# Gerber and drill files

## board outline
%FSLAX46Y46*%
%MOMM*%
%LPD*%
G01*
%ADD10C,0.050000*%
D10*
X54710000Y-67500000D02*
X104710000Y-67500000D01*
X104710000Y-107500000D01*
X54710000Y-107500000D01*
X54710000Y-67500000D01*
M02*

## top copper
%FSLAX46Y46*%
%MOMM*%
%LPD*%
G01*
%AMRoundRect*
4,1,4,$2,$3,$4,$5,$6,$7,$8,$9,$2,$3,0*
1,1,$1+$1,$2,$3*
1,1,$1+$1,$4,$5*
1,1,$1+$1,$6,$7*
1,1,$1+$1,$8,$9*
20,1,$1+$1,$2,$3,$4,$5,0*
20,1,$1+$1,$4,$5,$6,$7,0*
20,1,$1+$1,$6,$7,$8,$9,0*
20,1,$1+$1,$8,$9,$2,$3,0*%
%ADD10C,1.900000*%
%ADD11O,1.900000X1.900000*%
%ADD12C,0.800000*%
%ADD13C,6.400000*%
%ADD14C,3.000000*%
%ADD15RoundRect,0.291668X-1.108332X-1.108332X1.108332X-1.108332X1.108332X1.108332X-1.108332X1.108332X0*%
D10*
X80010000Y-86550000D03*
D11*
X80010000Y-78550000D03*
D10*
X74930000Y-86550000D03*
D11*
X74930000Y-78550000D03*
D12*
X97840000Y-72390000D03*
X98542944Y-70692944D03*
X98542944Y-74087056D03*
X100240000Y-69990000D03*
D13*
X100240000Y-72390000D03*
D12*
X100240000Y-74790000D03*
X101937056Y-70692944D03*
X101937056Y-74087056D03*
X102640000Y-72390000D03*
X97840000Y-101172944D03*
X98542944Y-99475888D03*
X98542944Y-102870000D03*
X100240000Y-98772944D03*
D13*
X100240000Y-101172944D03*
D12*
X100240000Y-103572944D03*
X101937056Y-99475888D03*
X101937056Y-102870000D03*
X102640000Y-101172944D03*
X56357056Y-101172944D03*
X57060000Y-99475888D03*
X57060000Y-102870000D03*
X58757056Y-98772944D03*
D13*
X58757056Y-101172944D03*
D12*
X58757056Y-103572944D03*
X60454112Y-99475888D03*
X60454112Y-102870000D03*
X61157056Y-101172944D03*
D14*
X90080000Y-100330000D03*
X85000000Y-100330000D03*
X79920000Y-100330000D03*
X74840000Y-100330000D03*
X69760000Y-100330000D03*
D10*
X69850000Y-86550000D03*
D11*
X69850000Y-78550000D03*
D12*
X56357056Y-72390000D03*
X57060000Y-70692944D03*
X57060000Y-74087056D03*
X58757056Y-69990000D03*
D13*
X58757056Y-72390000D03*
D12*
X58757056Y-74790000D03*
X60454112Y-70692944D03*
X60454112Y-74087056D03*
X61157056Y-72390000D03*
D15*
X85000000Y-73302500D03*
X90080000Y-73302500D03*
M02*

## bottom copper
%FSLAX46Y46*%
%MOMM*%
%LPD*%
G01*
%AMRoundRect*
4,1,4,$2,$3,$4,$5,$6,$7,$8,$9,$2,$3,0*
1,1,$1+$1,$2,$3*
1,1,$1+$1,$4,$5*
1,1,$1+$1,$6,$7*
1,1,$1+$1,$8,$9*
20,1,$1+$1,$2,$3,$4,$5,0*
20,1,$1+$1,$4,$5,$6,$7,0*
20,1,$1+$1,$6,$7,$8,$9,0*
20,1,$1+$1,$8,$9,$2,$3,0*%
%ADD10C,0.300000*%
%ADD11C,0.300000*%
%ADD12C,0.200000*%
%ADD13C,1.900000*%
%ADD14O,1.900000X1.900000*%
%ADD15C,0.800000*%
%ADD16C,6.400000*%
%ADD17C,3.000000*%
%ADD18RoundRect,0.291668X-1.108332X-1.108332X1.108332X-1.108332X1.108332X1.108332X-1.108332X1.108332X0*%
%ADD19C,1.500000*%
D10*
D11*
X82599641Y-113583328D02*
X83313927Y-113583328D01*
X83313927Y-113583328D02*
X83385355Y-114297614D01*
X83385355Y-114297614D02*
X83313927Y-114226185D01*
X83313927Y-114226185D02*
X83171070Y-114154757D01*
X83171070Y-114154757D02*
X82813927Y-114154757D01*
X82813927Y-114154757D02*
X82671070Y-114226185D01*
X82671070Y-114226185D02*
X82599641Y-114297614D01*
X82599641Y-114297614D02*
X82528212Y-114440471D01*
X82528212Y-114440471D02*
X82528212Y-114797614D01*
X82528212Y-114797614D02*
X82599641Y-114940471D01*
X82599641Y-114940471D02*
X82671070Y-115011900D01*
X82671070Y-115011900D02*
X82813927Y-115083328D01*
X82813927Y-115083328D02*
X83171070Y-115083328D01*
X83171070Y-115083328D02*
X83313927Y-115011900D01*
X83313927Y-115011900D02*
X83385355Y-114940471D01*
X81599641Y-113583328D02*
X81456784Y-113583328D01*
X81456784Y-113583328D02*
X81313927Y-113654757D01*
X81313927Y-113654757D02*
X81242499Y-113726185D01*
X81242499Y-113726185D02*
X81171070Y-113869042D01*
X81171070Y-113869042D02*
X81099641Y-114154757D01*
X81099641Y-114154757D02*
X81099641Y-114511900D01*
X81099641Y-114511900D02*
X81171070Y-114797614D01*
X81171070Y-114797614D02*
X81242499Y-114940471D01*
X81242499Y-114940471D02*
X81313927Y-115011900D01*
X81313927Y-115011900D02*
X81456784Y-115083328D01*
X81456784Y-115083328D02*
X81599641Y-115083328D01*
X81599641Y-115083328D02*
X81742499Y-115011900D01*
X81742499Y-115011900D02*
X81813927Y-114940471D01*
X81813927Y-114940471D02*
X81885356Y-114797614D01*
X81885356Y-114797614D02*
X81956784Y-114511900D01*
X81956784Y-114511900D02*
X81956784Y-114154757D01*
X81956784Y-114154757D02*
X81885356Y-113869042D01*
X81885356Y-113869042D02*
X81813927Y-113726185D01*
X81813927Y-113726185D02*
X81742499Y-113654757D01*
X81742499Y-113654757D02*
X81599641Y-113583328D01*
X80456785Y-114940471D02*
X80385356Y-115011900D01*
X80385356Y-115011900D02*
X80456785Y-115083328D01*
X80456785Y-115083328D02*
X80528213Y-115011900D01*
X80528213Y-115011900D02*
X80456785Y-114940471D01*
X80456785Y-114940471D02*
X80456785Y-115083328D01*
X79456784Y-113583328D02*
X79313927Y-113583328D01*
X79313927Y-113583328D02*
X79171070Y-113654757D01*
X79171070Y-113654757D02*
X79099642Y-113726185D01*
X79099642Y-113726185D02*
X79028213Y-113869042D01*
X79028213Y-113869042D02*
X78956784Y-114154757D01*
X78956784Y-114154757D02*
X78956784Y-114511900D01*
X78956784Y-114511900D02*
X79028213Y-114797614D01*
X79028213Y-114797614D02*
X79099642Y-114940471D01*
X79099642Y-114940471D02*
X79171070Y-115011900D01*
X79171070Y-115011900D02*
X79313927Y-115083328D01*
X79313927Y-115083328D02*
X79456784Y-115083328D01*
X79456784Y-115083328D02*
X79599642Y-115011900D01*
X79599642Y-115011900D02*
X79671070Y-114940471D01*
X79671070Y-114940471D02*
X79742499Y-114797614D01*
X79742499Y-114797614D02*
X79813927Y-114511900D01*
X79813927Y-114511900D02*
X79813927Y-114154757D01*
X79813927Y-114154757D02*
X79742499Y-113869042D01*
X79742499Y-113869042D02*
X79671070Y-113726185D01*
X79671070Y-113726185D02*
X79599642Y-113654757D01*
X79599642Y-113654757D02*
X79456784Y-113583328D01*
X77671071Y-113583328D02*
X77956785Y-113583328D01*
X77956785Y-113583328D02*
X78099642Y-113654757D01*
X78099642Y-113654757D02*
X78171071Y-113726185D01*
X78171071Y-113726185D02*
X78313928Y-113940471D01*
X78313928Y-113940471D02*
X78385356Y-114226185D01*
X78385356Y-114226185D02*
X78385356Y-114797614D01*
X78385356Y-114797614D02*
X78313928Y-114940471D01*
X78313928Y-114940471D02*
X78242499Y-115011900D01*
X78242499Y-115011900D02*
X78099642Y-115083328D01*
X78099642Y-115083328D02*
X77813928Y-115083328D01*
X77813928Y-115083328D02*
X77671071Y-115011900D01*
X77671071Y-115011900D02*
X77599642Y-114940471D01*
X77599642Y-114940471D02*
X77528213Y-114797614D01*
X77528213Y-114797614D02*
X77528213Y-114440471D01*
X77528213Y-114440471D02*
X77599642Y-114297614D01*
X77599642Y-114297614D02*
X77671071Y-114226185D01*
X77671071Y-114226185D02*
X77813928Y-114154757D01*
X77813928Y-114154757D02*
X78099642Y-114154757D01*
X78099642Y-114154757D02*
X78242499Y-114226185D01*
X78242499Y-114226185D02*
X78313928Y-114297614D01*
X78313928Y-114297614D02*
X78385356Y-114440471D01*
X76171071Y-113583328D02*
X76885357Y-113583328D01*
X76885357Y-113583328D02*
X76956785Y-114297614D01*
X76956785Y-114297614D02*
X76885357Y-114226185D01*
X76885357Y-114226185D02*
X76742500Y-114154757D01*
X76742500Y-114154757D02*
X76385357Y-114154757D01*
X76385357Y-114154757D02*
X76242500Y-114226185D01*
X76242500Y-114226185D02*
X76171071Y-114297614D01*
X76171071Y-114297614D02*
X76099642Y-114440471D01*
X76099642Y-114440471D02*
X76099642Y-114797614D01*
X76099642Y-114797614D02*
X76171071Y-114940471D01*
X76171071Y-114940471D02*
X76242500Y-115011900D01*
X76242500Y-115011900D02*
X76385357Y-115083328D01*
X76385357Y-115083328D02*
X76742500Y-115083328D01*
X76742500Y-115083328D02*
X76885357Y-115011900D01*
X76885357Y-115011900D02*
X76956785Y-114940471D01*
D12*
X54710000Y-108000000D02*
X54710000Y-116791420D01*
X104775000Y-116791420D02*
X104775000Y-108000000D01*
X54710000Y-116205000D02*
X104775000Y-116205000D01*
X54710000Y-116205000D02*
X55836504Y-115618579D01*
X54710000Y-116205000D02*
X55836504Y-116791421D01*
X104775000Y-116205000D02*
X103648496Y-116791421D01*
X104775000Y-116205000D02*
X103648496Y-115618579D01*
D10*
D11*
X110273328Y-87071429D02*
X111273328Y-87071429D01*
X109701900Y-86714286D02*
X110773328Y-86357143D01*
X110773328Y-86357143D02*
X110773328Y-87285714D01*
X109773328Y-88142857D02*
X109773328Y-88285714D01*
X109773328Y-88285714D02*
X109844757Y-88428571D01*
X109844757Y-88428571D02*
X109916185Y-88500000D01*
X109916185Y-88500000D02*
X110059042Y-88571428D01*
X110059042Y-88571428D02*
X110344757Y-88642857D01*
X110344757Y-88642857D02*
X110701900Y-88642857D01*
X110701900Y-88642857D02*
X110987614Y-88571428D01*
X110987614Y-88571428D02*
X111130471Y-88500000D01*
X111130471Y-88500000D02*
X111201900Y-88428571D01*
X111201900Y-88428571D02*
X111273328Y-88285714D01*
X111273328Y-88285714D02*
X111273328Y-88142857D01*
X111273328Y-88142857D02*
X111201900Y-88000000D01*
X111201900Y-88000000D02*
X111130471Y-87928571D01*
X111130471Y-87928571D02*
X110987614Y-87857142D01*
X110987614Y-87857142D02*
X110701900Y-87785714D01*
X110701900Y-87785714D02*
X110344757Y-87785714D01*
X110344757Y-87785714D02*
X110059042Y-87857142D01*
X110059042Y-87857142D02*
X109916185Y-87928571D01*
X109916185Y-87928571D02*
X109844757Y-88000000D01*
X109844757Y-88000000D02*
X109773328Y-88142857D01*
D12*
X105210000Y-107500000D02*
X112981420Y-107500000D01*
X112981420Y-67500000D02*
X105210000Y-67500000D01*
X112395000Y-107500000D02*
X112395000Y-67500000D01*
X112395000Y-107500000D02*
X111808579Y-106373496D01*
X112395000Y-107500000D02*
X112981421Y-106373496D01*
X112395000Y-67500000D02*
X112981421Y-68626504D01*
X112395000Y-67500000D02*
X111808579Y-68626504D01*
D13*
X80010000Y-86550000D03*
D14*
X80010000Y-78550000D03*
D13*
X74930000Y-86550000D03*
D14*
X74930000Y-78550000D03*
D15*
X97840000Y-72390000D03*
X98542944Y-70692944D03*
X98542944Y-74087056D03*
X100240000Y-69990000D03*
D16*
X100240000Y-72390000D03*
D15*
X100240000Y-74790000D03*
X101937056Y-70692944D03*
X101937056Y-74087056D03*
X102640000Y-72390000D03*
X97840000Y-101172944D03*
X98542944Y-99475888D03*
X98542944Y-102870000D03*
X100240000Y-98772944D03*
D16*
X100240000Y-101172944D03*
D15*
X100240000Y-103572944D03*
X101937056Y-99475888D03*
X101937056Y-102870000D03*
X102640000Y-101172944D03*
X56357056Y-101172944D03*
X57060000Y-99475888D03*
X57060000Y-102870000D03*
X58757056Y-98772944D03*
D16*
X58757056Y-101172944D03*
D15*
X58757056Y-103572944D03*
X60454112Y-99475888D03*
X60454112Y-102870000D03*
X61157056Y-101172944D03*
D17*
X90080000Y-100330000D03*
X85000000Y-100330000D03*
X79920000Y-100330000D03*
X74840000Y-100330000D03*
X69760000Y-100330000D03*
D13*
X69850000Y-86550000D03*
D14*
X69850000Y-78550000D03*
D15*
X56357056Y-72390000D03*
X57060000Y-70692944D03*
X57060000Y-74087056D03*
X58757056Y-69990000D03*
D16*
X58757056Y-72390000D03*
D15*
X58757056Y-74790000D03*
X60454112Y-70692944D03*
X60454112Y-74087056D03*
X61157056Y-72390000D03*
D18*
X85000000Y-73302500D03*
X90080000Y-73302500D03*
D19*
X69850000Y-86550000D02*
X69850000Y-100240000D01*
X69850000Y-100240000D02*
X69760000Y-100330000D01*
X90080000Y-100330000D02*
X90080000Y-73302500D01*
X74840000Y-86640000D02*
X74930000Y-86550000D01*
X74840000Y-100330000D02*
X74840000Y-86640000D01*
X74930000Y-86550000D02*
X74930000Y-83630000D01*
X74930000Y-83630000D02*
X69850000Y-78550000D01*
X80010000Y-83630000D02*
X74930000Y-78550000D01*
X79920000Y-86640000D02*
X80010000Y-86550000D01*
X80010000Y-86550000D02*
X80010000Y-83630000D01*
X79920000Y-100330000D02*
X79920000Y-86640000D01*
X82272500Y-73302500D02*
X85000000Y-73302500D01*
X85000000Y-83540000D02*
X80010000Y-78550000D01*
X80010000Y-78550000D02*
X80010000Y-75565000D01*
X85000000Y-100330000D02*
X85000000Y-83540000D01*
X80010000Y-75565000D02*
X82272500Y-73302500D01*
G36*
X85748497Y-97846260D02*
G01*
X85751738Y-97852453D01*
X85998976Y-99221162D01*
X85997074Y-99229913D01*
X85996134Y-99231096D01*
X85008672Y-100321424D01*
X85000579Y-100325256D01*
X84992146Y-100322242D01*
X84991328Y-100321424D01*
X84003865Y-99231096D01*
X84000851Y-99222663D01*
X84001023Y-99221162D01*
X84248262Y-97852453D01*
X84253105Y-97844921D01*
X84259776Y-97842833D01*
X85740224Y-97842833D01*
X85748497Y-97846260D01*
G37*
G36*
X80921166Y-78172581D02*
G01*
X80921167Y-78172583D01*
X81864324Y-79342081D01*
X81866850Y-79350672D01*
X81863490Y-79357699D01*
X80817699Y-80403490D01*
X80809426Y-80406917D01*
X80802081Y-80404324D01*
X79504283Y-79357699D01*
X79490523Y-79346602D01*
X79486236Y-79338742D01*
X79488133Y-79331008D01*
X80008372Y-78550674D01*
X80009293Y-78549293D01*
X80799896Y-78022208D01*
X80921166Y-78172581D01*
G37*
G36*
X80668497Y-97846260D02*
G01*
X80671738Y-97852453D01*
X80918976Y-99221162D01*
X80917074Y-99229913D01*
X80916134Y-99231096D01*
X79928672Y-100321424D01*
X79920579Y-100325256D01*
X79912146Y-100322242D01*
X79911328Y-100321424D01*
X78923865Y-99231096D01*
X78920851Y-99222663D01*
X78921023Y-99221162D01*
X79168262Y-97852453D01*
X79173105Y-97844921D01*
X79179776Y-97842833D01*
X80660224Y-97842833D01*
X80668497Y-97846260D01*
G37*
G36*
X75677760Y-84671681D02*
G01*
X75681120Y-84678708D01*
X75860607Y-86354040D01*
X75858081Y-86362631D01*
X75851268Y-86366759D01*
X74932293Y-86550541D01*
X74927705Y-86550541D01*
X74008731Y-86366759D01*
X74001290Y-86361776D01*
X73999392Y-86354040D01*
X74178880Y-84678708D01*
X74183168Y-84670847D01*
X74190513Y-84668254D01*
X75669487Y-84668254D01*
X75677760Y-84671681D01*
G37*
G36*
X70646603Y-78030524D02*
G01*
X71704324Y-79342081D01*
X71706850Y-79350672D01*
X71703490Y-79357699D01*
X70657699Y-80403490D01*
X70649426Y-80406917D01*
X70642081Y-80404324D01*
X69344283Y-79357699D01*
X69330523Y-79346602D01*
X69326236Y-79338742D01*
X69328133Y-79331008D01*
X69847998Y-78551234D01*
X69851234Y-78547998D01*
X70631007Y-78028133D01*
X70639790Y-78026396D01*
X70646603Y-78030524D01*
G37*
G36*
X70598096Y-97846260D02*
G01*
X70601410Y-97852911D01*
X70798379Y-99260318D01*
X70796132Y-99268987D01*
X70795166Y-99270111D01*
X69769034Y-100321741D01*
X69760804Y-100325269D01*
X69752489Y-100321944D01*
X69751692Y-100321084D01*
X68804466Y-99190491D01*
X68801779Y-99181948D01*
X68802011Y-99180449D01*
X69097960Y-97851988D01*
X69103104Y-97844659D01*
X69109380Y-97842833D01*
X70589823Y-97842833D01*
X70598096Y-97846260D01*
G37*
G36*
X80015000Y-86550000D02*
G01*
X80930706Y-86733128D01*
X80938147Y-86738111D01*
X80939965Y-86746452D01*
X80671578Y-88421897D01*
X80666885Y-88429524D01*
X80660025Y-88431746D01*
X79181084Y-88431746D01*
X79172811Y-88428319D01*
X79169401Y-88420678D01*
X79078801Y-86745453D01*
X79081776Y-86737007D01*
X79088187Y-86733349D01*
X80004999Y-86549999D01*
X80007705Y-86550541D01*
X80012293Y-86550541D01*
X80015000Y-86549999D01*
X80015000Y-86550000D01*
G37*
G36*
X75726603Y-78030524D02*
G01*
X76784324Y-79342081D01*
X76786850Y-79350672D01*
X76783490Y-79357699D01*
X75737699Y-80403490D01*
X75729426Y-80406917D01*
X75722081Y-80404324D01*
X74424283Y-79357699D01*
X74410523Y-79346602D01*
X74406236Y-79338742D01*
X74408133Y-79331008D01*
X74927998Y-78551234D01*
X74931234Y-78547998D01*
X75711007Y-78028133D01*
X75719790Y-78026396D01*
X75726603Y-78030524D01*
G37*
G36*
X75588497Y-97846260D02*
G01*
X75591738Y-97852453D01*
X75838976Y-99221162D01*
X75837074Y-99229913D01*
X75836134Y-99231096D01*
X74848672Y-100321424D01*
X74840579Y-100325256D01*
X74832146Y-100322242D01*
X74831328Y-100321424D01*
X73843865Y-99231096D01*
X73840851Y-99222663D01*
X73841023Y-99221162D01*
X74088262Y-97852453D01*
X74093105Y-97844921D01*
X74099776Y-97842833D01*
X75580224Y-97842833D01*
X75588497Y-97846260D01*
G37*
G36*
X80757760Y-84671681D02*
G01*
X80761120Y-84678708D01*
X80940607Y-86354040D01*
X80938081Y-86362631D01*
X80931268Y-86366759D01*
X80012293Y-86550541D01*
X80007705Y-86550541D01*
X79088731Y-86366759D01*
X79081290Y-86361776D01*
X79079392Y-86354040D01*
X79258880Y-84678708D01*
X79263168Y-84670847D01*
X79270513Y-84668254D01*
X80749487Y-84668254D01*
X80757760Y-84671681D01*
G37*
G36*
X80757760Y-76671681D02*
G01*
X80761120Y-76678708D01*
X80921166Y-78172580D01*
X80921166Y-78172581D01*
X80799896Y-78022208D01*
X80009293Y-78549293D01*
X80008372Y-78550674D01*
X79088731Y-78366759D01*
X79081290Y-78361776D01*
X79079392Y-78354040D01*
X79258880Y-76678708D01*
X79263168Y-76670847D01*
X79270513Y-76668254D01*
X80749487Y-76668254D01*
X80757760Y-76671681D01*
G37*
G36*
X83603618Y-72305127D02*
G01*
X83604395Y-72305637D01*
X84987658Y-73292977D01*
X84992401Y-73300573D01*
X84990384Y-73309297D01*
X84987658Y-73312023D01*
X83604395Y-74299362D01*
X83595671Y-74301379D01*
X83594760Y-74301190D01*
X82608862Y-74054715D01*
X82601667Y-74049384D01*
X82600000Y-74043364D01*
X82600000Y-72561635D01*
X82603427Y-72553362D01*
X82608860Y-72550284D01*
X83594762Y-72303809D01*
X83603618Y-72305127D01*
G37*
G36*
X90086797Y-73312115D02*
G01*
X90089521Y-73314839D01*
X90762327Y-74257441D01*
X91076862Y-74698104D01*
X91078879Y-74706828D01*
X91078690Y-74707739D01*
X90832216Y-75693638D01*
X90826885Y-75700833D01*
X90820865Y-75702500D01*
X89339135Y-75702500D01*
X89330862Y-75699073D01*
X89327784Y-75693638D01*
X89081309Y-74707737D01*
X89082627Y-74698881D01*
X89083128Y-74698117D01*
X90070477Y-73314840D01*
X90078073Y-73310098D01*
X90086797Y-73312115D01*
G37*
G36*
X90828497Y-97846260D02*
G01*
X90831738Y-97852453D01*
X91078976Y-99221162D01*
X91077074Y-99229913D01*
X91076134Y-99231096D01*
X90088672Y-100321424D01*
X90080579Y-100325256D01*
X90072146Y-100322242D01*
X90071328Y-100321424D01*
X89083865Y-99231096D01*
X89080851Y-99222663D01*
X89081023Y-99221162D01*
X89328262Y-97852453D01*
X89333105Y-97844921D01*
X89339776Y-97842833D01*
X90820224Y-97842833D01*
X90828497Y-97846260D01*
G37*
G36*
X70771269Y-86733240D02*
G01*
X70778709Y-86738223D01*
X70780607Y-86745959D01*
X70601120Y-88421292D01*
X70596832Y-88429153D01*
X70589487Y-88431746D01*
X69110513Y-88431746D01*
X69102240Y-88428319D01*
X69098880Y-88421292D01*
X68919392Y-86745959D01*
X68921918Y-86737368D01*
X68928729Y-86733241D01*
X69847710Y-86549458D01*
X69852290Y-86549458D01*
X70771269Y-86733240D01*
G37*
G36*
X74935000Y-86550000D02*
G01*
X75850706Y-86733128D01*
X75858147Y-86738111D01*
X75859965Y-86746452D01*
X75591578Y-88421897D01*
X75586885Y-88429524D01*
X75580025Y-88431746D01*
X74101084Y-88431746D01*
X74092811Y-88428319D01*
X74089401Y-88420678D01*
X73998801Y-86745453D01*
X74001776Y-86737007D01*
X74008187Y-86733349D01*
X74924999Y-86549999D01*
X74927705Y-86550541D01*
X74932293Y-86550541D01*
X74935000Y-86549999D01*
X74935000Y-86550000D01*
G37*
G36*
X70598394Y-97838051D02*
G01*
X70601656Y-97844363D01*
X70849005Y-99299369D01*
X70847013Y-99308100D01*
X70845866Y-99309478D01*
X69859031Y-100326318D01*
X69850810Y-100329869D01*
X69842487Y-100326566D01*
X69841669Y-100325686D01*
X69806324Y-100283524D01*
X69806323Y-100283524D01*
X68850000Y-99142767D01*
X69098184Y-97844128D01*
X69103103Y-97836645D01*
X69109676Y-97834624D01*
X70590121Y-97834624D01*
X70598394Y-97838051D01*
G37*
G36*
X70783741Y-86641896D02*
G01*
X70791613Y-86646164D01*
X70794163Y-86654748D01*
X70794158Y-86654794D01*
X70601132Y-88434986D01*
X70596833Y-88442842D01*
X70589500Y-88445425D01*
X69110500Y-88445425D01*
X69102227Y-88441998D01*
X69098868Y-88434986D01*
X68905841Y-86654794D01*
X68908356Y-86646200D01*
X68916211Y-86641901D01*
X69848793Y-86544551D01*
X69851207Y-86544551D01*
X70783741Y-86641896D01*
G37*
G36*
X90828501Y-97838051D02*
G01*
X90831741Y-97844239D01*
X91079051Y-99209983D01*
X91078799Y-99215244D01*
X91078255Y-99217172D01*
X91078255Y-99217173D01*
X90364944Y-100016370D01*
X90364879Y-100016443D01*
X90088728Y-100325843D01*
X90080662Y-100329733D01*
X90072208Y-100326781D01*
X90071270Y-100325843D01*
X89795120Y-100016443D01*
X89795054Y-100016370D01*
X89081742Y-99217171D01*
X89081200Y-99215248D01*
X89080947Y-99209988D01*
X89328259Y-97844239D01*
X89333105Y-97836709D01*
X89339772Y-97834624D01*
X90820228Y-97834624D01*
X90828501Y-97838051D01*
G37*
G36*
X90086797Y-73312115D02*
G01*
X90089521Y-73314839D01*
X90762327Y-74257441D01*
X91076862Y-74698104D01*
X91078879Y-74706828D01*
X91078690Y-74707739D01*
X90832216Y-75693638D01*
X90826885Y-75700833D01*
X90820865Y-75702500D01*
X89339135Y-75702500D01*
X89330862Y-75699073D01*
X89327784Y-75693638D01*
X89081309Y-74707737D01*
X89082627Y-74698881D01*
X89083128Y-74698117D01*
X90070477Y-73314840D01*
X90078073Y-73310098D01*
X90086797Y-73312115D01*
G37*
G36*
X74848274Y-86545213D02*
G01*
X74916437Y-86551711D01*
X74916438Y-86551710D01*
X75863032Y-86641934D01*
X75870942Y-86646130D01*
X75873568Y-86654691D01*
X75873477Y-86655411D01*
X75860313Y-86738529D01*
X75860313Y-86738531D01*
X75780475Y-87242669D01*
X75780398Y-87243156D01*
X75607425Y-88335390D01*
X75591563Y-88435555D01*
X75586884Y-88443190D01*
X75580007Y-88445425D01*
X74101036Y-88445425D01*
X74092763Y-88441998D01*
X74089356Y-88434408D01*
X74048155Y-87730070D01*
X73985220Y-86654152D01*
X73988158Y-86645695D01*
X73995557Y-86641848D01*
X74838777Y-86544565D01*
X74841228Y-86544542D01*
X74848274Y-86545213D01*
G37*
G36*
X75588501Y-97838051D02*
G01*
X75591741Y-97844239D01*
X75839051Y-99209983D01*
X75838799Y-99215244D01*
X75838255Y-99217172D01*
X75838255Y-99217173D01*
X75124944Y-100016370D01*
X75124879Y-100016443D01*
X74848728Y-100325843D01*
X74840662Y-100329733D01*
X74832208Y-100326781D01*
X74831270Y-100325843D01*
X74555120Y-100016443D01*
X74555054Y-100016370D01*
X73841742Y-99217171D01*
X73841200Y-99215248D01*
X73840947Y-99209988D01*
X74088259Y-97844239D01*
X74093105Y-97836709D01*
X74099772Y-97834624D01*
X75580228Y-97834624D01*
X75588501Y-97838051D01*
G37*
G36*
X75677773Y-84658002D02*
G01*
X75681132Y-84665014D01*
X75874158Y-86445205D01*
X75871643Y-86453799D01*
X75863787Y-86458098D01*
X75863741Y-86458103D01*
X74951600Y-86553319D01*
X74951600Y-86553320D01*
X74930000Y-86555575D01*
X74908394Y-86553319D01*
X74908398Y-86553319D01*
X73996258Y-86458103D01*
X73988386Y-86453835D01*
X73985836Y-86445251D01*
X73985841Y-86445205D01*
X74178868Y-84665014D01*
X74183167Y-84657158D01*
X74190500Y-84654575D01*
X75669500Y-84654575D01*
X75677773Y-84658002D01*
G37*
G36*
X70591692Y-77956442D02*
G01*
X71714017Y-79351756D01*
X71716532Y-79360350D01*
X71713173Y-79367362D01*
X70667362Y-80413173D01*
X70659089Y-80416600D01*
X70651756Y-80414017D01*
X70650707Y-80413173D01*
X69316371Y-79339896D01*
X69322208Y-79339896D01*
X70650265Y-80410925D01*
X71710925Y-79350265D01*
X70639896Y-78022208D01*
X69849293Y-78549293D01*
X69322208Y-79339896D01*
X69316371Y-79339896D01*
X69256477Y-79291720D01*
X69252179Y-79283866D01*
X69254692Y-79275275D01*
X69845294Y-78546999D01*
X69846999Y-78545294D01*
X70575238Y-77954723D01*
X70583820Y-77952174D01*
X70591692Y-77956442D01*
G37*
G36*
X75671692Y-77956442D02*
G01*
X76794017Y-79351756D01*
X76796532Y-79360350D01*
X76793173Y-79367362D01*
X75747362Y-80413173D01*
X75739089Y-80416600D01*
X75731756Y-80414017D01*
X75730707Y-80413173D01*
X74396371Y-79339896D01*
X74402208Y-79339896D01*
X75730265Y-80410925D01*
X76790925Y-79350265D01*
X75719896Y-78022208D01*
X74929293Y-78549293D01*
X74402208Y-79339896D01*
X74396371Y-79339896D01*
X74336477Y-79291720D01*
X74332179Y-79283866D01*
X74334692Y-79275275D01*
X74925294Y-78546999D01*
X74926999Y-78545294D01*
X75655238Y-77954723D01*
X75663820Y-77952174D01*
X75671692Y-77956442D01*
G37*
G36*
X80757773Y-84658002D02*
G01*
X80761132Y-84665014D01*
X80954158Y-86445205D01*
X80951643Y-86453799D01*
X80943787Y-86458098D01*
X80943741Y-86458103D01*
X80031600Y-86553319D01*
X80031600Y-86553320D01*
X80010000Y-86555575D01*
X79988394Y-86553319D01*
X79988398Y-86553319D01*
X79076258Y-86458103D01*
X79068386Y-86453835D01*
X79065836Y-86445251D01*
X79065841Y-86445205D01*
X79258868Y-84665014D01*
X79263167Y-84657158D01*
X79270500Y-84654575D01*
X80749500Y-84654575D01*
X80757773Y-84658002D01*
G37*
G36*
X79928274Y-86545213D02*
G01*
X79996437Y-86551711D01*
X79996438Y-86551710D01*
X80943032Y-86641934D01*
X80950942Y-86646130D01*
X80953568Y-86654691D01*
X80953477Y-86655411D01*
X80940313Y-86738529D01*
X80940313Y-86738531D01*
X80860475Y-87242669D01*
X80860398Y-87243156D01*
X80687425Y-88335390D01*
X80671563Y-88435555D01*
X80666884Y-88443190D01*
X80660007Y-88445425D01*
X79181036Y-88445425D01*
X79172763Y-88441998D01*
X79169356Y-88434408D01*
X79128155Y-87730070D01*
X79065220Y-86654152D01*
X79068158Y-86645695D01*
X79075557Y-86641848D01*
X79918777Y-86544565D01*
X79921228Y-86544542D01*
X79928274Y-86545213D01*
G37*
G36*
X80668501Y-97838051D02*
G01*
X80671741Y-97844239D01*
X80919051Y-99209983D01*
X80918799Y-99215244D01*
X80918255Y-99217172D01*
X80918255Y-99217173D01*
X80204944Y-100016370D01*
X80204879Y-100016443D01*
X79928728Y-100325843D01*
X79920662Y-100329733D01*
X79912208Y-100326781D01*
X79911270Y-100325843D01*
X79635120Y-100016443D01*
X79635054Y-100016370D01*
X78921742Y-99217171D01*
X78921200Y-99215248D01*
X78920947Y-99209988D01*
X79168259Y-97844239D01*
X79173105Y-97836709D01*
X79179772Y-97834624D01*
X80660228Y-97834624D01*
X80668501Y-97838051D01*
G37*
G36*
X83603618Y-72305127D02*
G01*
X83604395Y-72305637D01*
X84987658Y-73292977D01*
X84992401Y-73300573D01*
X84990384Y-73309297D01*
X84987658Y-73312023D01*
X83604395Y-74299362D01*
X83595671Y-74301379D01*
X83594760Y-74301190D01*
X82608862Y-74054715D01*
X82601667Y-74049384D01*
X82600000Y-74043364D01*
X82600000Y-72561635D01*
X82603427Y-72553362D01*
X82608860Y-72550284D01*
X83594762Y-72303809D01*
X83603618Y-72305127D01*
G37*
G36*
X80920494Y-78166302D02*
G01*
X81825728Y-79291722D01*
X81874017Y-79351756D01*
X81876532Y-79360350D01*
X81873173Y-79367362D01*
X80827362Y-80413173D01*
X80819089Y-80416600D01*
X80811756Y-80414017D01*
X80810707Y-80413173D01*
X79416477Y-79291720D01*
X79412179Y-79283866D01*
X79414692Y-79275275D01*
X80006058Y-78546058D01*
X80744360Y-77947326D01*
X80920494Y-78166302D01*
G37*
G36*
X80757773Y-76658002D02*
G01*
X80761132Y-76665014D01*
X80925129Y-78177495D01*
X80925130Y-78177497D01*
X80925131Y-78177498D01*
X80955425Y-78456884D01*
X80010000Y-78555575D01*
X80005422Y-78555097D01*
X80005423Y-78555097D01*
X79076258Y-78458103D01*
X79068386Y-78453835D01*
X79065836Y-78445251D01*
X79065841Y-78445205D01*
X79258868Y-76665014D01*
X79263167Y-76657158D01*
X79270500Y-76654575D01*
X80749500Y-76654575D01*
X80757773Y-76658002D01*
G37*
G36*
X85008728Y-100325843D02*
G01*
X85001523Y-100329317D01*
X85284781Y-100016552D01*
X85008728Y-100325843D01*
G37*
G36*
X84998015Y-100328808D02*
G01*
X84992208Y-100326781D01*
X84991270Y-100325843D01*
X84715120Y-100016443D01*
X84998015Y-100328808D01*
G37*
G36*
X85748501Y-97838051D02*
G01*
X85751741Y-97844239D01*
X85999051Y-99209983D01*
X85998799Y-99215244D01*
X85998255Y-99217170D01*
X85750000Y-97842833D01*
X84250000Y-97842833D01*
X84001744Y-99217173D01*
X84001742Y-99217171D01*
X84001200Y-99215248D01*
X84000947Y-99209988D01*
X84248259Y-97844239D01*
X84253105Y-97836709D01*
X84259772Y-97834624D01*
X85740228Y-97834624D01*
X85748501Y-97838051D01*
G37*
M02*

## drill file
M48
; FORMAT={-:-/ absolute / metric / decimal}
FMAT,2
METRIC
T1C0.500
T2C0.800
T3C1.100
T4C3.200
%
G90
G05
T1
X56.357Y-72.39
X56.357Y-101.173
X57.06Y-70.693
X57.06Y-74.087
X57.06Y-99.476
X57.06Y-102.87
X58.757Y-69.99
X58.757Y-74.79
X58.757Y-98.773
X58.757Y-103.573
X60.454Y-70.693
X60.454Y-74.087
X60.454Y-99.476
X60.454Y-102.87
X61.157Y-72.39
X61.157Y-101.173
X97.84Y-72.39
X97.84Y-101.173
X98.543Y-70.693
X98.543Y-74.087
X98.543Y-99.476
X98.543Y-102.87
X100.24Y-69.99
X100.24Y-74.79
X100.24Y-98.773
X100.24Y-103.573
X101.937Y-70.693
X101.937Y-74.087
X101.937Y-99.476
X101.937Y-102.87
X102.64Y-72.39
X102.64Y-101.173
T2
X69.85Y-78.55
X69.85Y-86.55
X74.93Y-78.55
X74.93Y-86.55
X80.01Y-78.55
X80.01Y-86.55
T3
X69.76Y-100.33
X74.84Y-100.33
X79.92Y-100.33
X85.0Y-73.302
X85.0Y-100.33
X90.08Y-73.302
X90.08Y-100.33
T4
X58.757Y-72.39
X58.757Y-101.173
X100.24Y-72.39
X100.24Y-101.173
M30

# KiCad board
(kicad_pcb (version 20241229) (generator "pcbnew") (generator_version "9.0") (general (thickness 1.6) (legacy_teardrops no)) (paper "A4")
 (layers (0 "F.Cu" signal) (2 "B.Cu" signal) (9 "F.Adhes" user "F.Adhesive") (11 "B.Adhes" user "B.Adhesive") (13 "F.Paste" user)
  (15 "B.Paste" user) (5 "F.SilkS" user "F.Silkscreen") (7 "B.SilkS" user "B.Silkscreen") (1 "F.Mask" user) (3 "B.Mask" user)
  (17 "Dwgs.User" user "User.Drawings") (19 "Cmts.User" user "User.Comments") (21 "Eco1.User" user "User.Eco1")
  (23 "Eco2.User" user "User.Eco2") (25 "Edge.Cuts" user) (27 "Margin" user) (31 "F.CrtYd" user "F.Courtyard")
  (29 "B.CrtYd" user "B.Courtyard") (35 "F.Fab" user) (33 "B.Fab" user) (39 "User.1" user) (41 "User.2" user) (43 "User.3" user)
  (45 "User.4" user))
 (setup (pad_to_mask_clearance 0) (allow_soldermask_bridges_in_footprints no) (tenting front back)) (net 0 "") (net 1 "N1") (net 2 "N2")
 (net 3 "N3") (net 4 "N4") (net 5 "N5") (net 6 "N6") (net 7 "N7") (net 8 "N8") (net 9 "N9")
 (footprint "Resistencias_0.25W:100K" (layer "F.Cu") (at 80.01 86.55 90)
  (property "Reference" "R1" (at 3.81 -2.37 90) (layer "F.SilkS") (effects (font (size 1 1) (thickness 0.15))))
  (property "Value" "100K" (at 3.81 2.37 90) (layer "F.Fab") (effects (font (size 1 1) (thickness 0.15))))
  (pad "1" thru_hole circle (at 0 0 90) (size 1.9 1.9) (drill 0.8) (layers "*.Cu" "*.Mask") (remove_unused_layers no) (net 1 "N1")
   (teardrops (best_length_ratio 0.5) (max_length 1) (best_width_ratio 1) (max_width 2) (curved_edges no) (filter_ratio 0.9) (enabled yes)
    (allow_two_segments yes) (prefer_zone_connections yes)))
  (pad "2" thru_hole oval (at 8 0 90) (size 1.9 1.9) (drill 0.8) (layers "*.Cu" "*.Mask") (remove_unused_layers no) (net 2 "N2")
   (teardrops (best_length_ratio 0.5) (max_length 1) (best_width_ratio 1) (max_width 2) (curved_edges no) (filter_ratio 0.9) (enabled yes)
    (allow_two_segments yes) (prefer_zone_connections yes))))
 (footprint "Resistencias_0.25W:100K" (layer "F.Cu") (at 74.93 86.55 90)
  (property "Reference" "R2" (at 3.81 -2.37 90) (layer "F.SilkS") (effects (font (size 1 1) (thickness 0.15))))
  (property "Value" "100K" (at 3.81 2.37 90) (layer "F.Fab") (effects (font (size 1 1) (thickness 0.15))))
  (pad "1" thru_hole circle (at 0 0 90) (size 1.9 1.9) (drill 0.8) (layers "*.Cu" "*.Mask") (remove_unused_layers no) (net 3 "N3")
   (teardrops (best_length_ratio 0.5) (max_length 1) (best_width_ratio 1) (max_width 2) (curved_edges no) (filter_ratio 0.9) (enabled yes)
    (allow_two_segments yes) (prefer_zone_connections yes)))
  (pad "2" thru_hole oval (at 8 0 90) (size 1.9 1.9) (drill 0.8) (layers "*.Cu" "*.Mask") (remove_unused_layers no) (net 1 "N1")
   (teardrops (best_length_ratio 0.5) (max_length 1) (best_width_ratio 1) (max_width 2) (curved_edges no) (filter_ratio 0.9) (enabled yes)
    (allow_two_segments yes) (prefer_zone_connections yes))))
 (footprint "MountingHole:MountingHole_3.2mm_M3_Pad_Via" (layer "F.Cu") (at 100.24 72.39)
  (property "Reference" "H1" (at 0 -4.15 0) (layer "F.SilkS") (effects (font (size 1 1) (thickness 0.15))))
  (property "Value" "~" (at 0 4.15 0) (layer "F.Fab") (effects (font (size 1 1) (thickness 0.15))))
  (pad "1" thru_hole circle (at -2.4 0) (size 0.8 0.8) (drill 0.5) (layers "*.Cu" "*.Mask") (remove_unused_layers no) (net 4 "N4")
   (zone_connect 2)
   (teardrops (best_length_ratio 0.5) (max_length 1) (best_width_ratio 1) (max_width 2) (curved_edges no) (filter_ratio 0.9) (enabled yes)
    (allow_two_segments yes) (prefer_zone_connections yes)))
  (pad "1" thru_hole circle (at -1.697056 -1.697056) (size 0.8 0.8) (drill 0.5) (layers "*.Cu" "*.Mask") (remove_unused_layers no)
   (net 4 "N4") (zone_connect 2)
   (teardrops (best_length_ratio 0.5) (max_length 1) (best_width_ratio 1) (max_width 2) (curved_edges no) (filter_ratio 0.9) (enabled yes)
    (allow_two_segments yes) (prefer_zone_connections yes)))
  (pad "1" thru_hole circle (at -1.697056 1.697056) (size 0.8 0.8) (drill 0.5) (layers "*.Cu" "*.Mask") (remove_unused_layers no)
   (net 4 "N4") (zone_connect 2)
   (teardrops (best_length_ratio 0.5) (max_length 1) (best_width_ratio 1) (max_width 2) (curved_edges no) (filter_ratio 0.9) (enabled yes)
    (allow_two_segments yes) (prefer_zone_connections yes)))
  (pad "1" thru_hole circle (at 0 -2.4) (size 0.8 0.8) (drill 0.5) (layers "*.Cu" "*.Mask") (remove_unused_layers no) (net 4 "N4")
   (zone_connect 2)
   (teardrops (best_length_ratio 0.5) (max_length 1) (best_width_ratio 1) (max_width 2) (curved_edges no) (filter_ratio 0.9) (enabled yes)
    (allow_two_segments yes) (prefer_zone_connections yes)))
  (pad "1" thru_hole circle (at 0 0) (size 6.4 6.4) (drill 3.2) (layers "*.Cu" "*.Mask") (remove_unused_layers no) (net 4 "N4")
   (zone_connect 2)
   (teardrops (best_length_ratio 0.5) (max_length 1) (best_width_ratio 1) (max_width 2) (curved_edges no) (filter_ratio 0.9) (enabled yes)
    (allow_two_segments yes) (prefer_zone_connections yes)))
  (pad "1" thru_hole circle (at 0 2.4) (size 0.8 0.8) (drill 0.5) (layers "*.Cu" "*.Mask") (remove_unused_layers no) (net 4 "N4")
   (zone_connect 2)
   (teardrops (best_length_ratio 0.5) (max_length 1) (best_width_ratio 1) (max_width 2) (curved_edges no) (filter_ratio 0.9) (enabled yes)
    (allow_two_segments yes) (prefer_zone_connections yes)))
  (pad "1" thru_hole circle (at 1.697056 -1.697056) (size 0.8 0.8) (drill 0.5) (layers "*.Cu" "*.Mask") (remove_unused_layers no)
   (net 4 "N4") (zone_connect 2)
   (teardrops (best_length_ratio 0.5) (max_length 1) (best_width_ratio 1) (max_width 2) (curved_edges no) (filter_ratio 0.9) (enabled yes)
    (allow_two_segments yes) (prefer_zone_connections yes)))
  (pad "1" thru_hole circle (at 1.697056 1.697056) (size 0.8 0.8) (drill 0.5) (layers "*.Cu" "*.Mask") (remove_unused_layers no)
   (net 4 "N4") (zone_connect 2)
   (teardrops (best_length_ratio 0.5) (max_length 1) (best_width_ratio 1) (max_width 2) (curved_edges no) (filter_ratio 0.9) (enabled yes)
    (allow_two_segments yes) (prefer_zone_connections yes)))
  (pad "1" thru_hole circle (at 2.4 0) (size 0.8 0.8) (drill 0.5) (layers "*.Cu" "*.Mask") (remove_unused_layers no) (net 4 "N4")
   (zone_connect 2)
   (teardrops (best_length_ratio 0.5) (max_length 1) (best_width_ratio 1) (max_width 2) (curved_edges no) (filter_ratio 0.9) (enabled yes)
    (allow_two_segments yes) (prefer_zone_connections yes))))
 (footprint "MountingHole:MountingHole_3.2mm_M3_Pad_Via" (layer "F.Cu") (at 100.24 101.172944)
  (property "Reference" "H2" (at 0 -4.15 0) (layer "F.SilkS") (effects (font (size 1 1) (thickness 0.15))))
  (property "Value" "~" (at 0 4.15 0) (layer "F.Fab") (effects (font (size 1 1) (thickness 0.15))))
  (pad "1" thru_hole circle (at -2.4 0) (size 0.8 0.8) (drill 0.5) (layers "*.Cu" "*.Mask") (remove_unused_layers no) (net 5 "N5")
   (zone_connect 2)
   (teardrops (best_length_ratio 0.5) (max_length 1) (best_width_ratio 1) (max_width 2) (curved_edges no) (filter_ratio 0.9) (enabled yes)
    (allow_two_segments yes) (prefer_zone_connections yes)))
  (pad "1" thru_hole circle (at -1.697056 -1.697056) (size 0.8 0.8) (drill 0.5) (layers "*.Cu" "*.Mask") (remove_unused_layers no)
   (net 5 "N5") (zone_connect 2)
   (teardrops (best_length_ratio 0.5) (max_length 1) (best_width_ratio 1) (max_width 2) (curved_edges no) (filter_ratio 0.9) (enabled yes)
    (allow_two_segments yes) (prefer_zone_connections yes)))
  (pad "1" thru_hole circle (at -1.697056 1.697056) (size 0.8 0.8) (drill 0.5) (layers "*.Cu" "*.Mask") (remove_unused_layers no)
   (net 5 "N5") (zone_connect 2)
   (teardrops (best_length_ratio 0.5) (max_length 1) (best_width_ratio 1) (max_width 2) (curved_edges no) (filter_ratio 0.9) (enabled yes)
    (allow_two_segments yes) (prefer_zone_connections yes)))
  (pad "1" thru_hole circle (at 0 -2.4) (size 0.8 0.8) (drill 0.5) (layers "*.Cu" "*.Mask") (remove_unused_layers no) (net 5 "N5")
   (zone_connect 2)
   (teardrops (best_length_ratio 0.5) (max_length 1) (best_width_ratio 1) (max_width 2) (curved_edges no) (filter_ratio 0.9) (enabled yes)
    (allow_two_segments yes) (prefer_zone_connections yes)))
  (pad "1" thru_hole circle (at 0 0) (size 6.4 6.4) (drill 3.2) (layers "*.Cu" "*.Mask") (remove_unused_layers no) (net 5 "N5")
   (zone_connect 2)
   (teardrops (best_length_ratio 0.5) (max_length 1) (best_width_ratio 1) (max_width 2) (curved_edges no) (filter_ratio 0.9) (enabled yes)
    (allow_two_segments yes) (prefer_zone_connections yes)))
  (pad "1" thru_hole circle (at 0 2.4) (size 0.8 0.8) (drill 0.5) (layers "*.Cu" "*.Mask") (remove_unused_layers no) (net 5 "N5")
   (zone_connect 2)
   (teardrops (best_length_ratio 0.5) (max_length 1) (best_width_ratio 1) (max_width 2) (curved_edges no) (filter_ratio 0.9) (enabled yes)
    (allow_two_segments yes) (prefer_zone_connections yes)))
  (pad "1" thru_hole circle (at 1.697056 -1.697056) (size 0.8 0.8) (drill 0.5) (layers "*.Cu" "*.Mask") (remove_unused_layers no)
   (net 5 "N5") (zone_connect 2)
   (teardrops (best_length_ratio 0.5) (max_length 1) (best_width_ratio 1) (max_width 2) (curved_edges no) (filter_ratio 0.9) (enabled yes)
    (allow_two_segments yes) (prefer_zone_connections yes)))
  (pad "1" thru_hole circle (at 1.697056 1.697056) (size 0.8 0.8) (drill 0.5) (layers "*.Cu" "*.Mask") (remove_unused_layers no)
   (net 5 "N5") (zone_connect 2)
   (teardrops (best_length_ratio 0.5) (max_length 1) (best_width_ratio 1) (max_width 2) (curved_edges no) (filter_ratio 0.9) (enabled yes)
    (allow_two_segments yes) (prefer_zone_connections yes)))
  (pad "1" thru_hole circle (at 2.4 0) (size 0.8 0.8) (drill 0.5) (layers "*.Cu" "*.Mask") (remove_unused_layers no) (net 5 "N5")
   (zone_connect 2)
   (teardrops (best_length_ratio 0.5) (max_length 1) (best_width_ratio 1) (max_width 2) (curved_edges no) (filter_ratio 0.9) (enabled yes)
    (allow_two_segments yes) (prefer_zone_connections yes))))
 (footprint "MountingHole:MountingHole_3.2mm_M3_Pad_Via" (layer "F.Cu") (at 58.757056 101.172944)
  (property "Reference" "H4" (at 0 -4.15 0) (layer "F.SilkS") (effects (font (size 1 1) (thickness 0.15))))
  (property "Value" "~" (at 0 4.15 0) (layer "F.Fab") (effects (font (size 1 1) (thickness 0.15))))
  (pad "1" thru_hole circle (at -2.4 0) (size 0.8 0.8) (drill 0.5) (layers "*.Cu" "*.Mask") (remove_unused_layers no) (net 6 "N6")
   (zone_connect 2)
   (teardrops (best_length_ratio 0.5) (max_length 1) (best_width_ratio 1) (max_width 2) (curved_edges no) (filter_ratio 0.9) (enabled yes)
    (allow_two_segments yes) (prefer_zone_connections yes)))
  (pad "1" thru_hole circle (at -1.697056 -1.697056) (size 0.8 0.8) (drill 0.5) (layers "*.Cu" "*.Mask") (remove_unused_layers no)
   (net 6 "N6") (zone_connect 2)
   (teardrops (best_length_ratio 0.5) (max_length 1) (best_width_ratio 1) (max_width 2) (curved_edges no) (filter_ratio 0.9) (enabled yes)
    (allow_two_segments yes) (prefer_zone_connections yes)))
  (pad "1" thru_hole circle (at -1.697056 1.697056) (size 0.8 0.8) (drill 0.5) (layers "*.Cu" "*.Mask") (remove_unused_layers no)
   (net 6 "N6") (zone_connect 2)
   (teardrops (best_length_ratio 0.5) (max_length 1) (best_width_ratio 1) (max_width 2) (curved_edges no) (filter_ratio 0.9) (enabled yes)
    (allow_two_segments yes) (prefer_zone_connections yes)))
  (pad "1" thru_hole circle (at 0 -2.4) (size 0.8 0.8) (drill 0.5) (layers "*.Cu" "*.Mask") (remove_unused_layers no) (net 6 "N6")
   (zone_connect 2)
   (teardrops (best_length_ratio 0.5) (max_length 1) (best_width_ratio 1) (max_width 2) (curved_edges no) (filter_ratio 0.9) (enabled yes)
    (allow_two_segments yes) (prefer_zone_connections yes)))
  (pad "1" thru_hole circle (at 0 0) (size 6.4 6.4) (drill 3.2) (layers "*.Cu" "*.Mask") (remove_unused_layers no) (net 6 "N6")
   (zone_connect 2)
   (teardrops (best_length_ratio 0.5) (max_length 1) (best_width_ratio 1) (max_width 2) (curved_edges no) (filter_ratio 0.9) (enabled yes)
    (allow_two_segments yes) (prefer_zone_connections yes)))
  (pad "1" thru_hole circle (at 0 2.4) (size 0.8 0.8) (drill 0.5) (layers "*.Cu" "*.Mask") (remove_unused_layers no) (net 6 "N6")
   (zone_connect 2)
   (teardrops (best_length_ratio 0.5) (max_length 1) (best_width_ratio 1) (max_width 2) (curved_edges no) (filter_ratio 0.9) (enabled yes)
    (allow_two_segments yes) (prefer_zone_connections yes)))
  (pad "1" thru_hole circle (at 1.697056 -1.697056) (size 0.8 0.8) (drill 0.5) (layers "*.Cu" "*.Mask") (remove_unused_layers no)
   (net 6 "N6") (zone_connect 2)
   (teardrops (best_length_ratio 0.5) (max_length 1) (best_width_ratio 1) (max_width 2) (curved_edges no) (filter_ratio 0.9) (enabled yes)
    (allow_two_segments yes) (prefer_zone_connections yes)))
  (pad "1" thru_hole circle (at 1.697056 1.697056) (size 0.8 0.8) (drill 0.5) (layers "*.Cu" "*.Mask") (remove_unused_layers no)
   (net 6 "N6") (zone_connect 2)
   (teardrops (best_length_ratio 0.5) (max_length 1) (best_width_ratio 1) (max_width 2) (curved_edges no) (filter_ratio 0.9) (enabled yes)
    (allow_two_segments yes) (prefer_zone_connections yes)))
  (pad "1" thru_hole circle (at 2.4 0) (size 0.8 0.8) (drill 0.5) (layers "*.Cu" "*.Mask") (remove_unused_layers no) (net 6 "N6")
   (zone_connect 2)
   (teardrops (best_length_ratio 0.5) (max_length 1) (best_width_ratio 1) (max_width 2) (curved_edges no) (filter_ratio 0.9) (enabled yes)
    (allow_two_segments yes) (prefer_zone_connections yes))))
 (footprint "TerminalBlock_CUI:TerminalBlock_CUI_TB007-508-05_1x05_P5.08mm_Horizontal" (layer "F.Cu") (at 90.08 100.33 180)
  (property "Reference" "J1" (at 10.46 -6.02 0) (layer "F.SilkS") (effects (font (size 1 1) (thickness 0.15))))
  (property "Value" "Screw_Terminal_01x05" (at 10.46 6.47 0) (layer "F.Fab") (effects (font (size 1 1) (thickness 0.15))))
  (pad "1" thru_hole circle (at 0 0 180) (size 3 3) (drill 1.1) (layers "*.Cu" "*.Mask") (remove_unused_layers no) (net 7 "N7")
   (teardrops (best_length_ratio 0.5) (max_length 1) (best_width_ratio 1) (max_width 2) (curved_edges no) (filter_ratio 0.9) (enabled yes)
    (allow_two_segments yes) (prefer_zone_connections yes)))
  (pad "2" thru_hole circle (at 5.08 0 180) (size 3 3) (drill 1.1) (layers "*.Cu" "*.Mask") (remove_unused_layers no) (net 2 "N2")
   (teardrops (best_length_ratio 0.5) (max_length 1) (best_width_ratio 1) (max_width 2) (curved_edges no) (filter_ratio 0.9) (enabled yes)
    (allow_two_segments yes) (prefer_zone_connections yes)))
  (pad "3" thru_hole circle (at 10.16 0 180) (size 3 3) (drill 1.1) (layers "*.Cu" "*.Mask") (remove_unused_layers no) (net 1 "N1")
   (teardrops (best_length_ratio 0.5) (max_length 1) (best_width_ratio 1) (max_width 2) (curved_edges no) (filter_ratio 0.9) (enabled yes)
    (allow_two_segments yes) (prefer_zone_connections yes)))
  (pad "4" thru_hole circle (at 15.24 0 180) (size 3 3) (drill 1.1) (layers "*.Cu" "*.Mask") (remove_unused_layers no) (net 3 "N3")
   (teardrops (best_length_ratio 0.5) (max_length 1) (best_width_ratio 1) (max_width 2) (curved_edges no) (filter_ratio 0.9) (enabled yes)
    (allow_two_segments yes) (prefer_zone_connections yes)))
  (pad "5" thru_hole circle (at 20.32 0 180) (size 3 3) (drill 1.1) (layers "*.Cu" "*.Mask") (remove_unused_layers no) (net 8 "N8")
   (teardrops (best_length_ratio 0.5) (max_length 1) (best_width_ratio 1) (max_width 2) (curved_edges no) (filter_ratio 0.9) (enabled yes)
    (allow_two_segments yes) (prefer_zone_connections yes))))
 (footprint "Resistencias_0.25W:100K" (layer "F.Cu") (at 69.85 86.55 90)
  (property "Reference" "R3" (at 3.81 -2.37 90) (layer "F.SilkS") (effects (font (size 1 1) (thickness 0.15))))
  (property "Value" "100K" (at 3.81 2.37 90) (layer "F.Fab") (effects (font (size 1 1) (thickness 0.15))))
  (pad "1" thru_hole circle (at 0 0 90) (size 1.9 1.9) (drill 0.8) (layers "*.Cu" "*.Mask") (remove_unused_layers no) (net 8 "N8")
   (teardrops (best_length_ratio 0.5) (max_length 1) (best_width_ratio 1) (max_width 2) (curved_edges no) (filter_ratio 0.9) (enabled yes)
    (allow_two_segments yes) (prefer_zone_connections yes)))
  (pad "2" thru_hole oval (at 8 0 90) (size 1.9 1.9) (drill 0.8) (layers "*.Cu" "*.Mask") (remove_unused_layers no) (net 3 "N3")
   (teardrops (best_length_ratio 0.5) (max_length 1) (best_width_ratio 1) (max_width 2) (curved_edges no) (filter_ratio 0.9) (enabled yes)
    (allow_two_segments yes) (prefer_zone_connections yes))))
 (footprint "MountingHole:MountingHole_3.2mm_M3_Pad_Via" (layer "F.Cu") (at 58.757056 72.39)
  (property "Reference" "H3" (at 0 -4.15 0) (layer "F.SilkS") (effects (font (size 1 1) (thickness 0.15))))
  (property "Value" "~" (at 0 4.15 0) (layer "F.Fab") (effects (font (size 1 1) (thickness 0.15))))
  (pad "1" thru_hole circle (at -2.4 0) (size 0.8 0.8) (drill 0.5) (layers "*.Cu" "*.Mask") (remove_unused_layers no) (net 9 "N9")
   (zone_connect 2)
   (teardrops (best_length_ratio 0.5) (max_length 1) (best_width_ratio 1) (max_width 2) (curved_edges no) (filter_ratio 0.9) (enabled yes)
    (allow_two_segments yes) (prefer_zone_connections yes)))
  (pad "1" thru_hole circle (at -1.697056 -1.697056) (size 0.8 0.8) (drill 0.5) (layers "*.Cu" "*.Mask") (remove_unused_layers no)
   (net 9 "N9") (zone_connect 2)
   (teardrops (best_length_ratio 0.5) (max_length 1) (best_width_ratio 1) (max_width 2) (curved_edges no) (filter_ratio 0.9) (enabled yes)
    (allow_two_segments yes) (prefer_zone_connections yes)))
  (pad "1" thru_hole circle (at -1.697056 1.697056) (size 0.8 0.8) (drill 0.5) (layers "*.Cu" "*.Mask") (remove_unused_layers no)
   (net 9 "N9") (zone_connect 2)
   (teardrops (best_length_ratio 0.5) (max_length 1) (best_width_ratio 1) (max_width 2) (curved_edges no) (filter_ratio 0.9) (enabled yes)
    (allow_two_segments yes) (prefer_zone_connections yes)))
  (pad "1" thru_hole circle (at 0 -2.4) (size 0.8 0.8) (drill 0.5) (layers "*.Cu" "*.Mask") (remove_unused_layers no) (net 9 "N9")
   (zone_connect 2)
   (teardrops (best_length_ratio 0.5) (max_length 1) (best_width_ratio 1) (max_width 2) (curved_edges no) (filter_ratio 0.9) (enabled yes)
    (allow_two_segments yes) (prefer_zone_connections yes)))
  (pad "1" thru_hole circle (at 0 0) (size 6.4 6.4) (drill 3.2) (layers "*.Cu" "*.Mask") (remove_unused_layers no) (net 9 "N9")
   (zone_connect 2)
   (teardrops (best_length_ratio 0.5) (max_length 1) (best_width_ratio 1) (max_width 2) (curved_edges no) (filter_ratio 0.9) (enabled yes)
    (allow_two_segments yes) (prefer_zone_connections yes)))
  (pad "1" thru_hole circle (at 0 2.4) (size 0.8 0.8) (drill 0.5) (layers "*.Cu" "*.Mask") (remove_unused_layers no) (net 9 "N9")
   (zone_connect 2)
   (teardrops (best_length_ratio 0.5) (max_length 1) (best_width_ratio 1) (max_width 2) (curved_edges no) (filter_ratio 0.9) (enabled yes)
    (allow_two_segments yes) (prefer_zone_connections yes)))
  (pad "1" thru_hole circle (at 1.697056 -1.697056) (size 0.8 0.8) (drill 0.5) (layers "*.Cu" "*.Mask") (remove_unused_layers no)
   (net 9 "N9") (zone_connect 2)
   (teardrops (best_length_ratio 0.5) (max_length 1) (best_width_ratio 1) (max_width 2) (curved_edges no) (filter_ratio 0.9) (enabled yes)
    (allow_two_segments yes) (prefer_zone_connections yes)))
  (pad "1" thru_hole circle (at 1.697056 1.697056) (size 0.8 0.8) (drill 0.5) (layers "*.Cu" "*.Mask") (remove_unused_layers no)
   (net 9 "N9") (zone_connect 2)
   (teardrops (best_length_ratio 0.5) (max_length 1) (best_width_ratio 1) (max_width 2) (curved_edges no) (filter_ratio 0.9) (enabled yes)
    (allow_two_segments yes) (prefer_zone_connections yes)))
  (pad "1" thru_hole circle (at 2.4 0) (size 0.8 0.8) (drill 0.5) (layers "*.Cu" "*.Mask") (remove_unused_layers no) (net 9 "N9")
   (zone_connect 2)
   (teardrops (best_length_ratio 0.5) (max_length 1) (best_width_ratio 1) (max_width 2) (curved_edges no) (filter_ratio 0.9) (enabled yes)
    (allow_two_segments yes) (prefer_zone_connections yes))))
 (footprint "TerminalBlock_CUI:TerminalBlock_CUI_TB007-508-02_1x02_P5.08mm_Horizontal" (layer "F.Cu") (at 85 73.3025)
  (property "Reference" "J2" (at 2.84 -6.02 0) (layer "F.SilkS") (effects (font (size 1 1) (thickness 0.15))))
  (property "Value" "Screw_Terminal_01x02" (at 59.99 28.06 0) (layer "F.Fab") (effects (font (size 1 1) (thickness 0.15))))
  (pad "1" thru_hole roundrect (at 0 0) (size 2.8 2.8) (drill 1.1) (layers "*.Cu" "*.Mask") (remove_unused_layers no)
   (roundrect_rratio 0.104167) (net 2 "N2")
   (teardrops (best_length_ratio 0.5) (max_length 1) (best_width_ratio 1) (max_width 2) (curved_edges no) (filter_ratio 0.9) (enabled yes)
    (allow_two_segments yes) (prefer_zone_connections yes)))
  (pad "2" thru_hole roundrect (at 5.08 0) (size 2.8 2.8) (drill 1.1) (layers "*.Cu" "*.Mask") (remove_unused_layers no)
   (roundrect_rratio 0.104167) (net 7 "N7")
   (teardrops (best_length_ratio 0.5) (max_length 1) (best_width_ratio 1) (max_width 2) (curved_edges no) (filter_ratio 0.9) (enabled yes)
    (allow_two_segments yes) (prefer_zone_connections yes))))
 (gr_rect (start 54.71 67.5) (end 104.71 107.5) (stroke (width 0.05) (type default)) (fill no) (layer "Edge.Cuts"))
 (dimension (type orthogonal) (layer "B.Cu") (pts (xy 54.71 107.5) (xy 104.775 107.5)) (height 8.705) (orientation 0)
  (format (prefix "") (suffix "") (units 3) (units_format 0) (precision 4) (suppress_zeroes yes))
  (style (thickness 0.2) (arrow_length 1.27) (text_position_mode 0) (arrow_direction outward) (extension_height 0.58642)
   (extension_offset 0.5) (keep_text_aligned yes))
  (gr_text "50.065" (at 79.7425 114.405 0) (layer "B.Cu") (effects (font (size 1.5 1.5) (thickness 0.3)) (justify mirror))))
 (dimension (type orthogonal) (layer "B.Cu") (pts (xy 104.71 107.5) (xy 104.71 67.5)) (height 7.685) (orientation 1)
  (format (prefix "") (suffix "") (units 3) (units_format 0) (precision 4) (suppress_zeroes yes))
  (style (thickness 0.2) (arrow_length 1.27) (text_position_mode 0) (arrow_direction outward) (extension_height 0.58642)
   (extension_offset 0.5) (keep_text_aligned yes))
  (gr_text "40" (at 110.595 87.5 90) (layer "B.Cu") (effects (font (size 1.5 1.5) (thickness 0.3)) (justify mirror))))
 (segment (start 69.85 86.55) (end 69.85 100.24) (width 1.5) (layer "B.Cu") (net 8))
 (segment (start 69.85 100.24) (end 69.76 100.33) (width 1.5) (layer "B.Cu") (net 8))
 (segment (start 90.08 100.33) (end 90.08 73.3025) (width 1.5) (layer "B.Cu") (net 7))
 (segment (start 74.84 86.64) (end 74.93 86.55) (width 1.5) (layer "B.Cu") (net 3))
 (segment (start 74.84 100.33) (end 74.84 86.64) (width 1.5) (layer "B.Cu") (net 3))
 (segment (start 74.93 86.55) (end 74.93 83.63) (width 1.5) (layer "B.Cu") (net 3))
 (segment (start 74.93 83.63) (end 69.85 78.55) (width 1.5) (layer "B.Cu") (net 3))
 (segment (start 80.01 83.63) (end 74.93 78.55) (width 1.5) (layer "B.Cu") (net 1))
 (segment (start 79.92 86.64) (end 80.01 86.55) (width 1.5) (layer "B.Cu") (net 1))
 (segment (start 80.01 86.55) (end 80.01 83.63) (width 1.5) (layer "B.Cu") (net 1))
 (segment (start 79.92 100.33) (end 79.92 86.64) (width 1.5) (layer "B.Cu") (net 1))
 (segment (start 82.2725 73.3025) (end 85 73.3025) (width 1.5) (layer "B.Cu") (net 2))
 (segment (start 85 83.54) (end 80.01 78.55) (width 1.5) (layer "B.Cu") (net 2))
 (segment (start 80.01 78.55) (end 80.01 75.565) (width 1.5) (layer "B.Cu") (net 2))
 (segment (start 85 100.33) (end 85 83.54) (width 1.5) (layer "B.Cu") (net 2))
 (segment (start 80.01 75.565) (end 82.2725 73.3025) (width 1.5) (layer "B.Cu") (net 2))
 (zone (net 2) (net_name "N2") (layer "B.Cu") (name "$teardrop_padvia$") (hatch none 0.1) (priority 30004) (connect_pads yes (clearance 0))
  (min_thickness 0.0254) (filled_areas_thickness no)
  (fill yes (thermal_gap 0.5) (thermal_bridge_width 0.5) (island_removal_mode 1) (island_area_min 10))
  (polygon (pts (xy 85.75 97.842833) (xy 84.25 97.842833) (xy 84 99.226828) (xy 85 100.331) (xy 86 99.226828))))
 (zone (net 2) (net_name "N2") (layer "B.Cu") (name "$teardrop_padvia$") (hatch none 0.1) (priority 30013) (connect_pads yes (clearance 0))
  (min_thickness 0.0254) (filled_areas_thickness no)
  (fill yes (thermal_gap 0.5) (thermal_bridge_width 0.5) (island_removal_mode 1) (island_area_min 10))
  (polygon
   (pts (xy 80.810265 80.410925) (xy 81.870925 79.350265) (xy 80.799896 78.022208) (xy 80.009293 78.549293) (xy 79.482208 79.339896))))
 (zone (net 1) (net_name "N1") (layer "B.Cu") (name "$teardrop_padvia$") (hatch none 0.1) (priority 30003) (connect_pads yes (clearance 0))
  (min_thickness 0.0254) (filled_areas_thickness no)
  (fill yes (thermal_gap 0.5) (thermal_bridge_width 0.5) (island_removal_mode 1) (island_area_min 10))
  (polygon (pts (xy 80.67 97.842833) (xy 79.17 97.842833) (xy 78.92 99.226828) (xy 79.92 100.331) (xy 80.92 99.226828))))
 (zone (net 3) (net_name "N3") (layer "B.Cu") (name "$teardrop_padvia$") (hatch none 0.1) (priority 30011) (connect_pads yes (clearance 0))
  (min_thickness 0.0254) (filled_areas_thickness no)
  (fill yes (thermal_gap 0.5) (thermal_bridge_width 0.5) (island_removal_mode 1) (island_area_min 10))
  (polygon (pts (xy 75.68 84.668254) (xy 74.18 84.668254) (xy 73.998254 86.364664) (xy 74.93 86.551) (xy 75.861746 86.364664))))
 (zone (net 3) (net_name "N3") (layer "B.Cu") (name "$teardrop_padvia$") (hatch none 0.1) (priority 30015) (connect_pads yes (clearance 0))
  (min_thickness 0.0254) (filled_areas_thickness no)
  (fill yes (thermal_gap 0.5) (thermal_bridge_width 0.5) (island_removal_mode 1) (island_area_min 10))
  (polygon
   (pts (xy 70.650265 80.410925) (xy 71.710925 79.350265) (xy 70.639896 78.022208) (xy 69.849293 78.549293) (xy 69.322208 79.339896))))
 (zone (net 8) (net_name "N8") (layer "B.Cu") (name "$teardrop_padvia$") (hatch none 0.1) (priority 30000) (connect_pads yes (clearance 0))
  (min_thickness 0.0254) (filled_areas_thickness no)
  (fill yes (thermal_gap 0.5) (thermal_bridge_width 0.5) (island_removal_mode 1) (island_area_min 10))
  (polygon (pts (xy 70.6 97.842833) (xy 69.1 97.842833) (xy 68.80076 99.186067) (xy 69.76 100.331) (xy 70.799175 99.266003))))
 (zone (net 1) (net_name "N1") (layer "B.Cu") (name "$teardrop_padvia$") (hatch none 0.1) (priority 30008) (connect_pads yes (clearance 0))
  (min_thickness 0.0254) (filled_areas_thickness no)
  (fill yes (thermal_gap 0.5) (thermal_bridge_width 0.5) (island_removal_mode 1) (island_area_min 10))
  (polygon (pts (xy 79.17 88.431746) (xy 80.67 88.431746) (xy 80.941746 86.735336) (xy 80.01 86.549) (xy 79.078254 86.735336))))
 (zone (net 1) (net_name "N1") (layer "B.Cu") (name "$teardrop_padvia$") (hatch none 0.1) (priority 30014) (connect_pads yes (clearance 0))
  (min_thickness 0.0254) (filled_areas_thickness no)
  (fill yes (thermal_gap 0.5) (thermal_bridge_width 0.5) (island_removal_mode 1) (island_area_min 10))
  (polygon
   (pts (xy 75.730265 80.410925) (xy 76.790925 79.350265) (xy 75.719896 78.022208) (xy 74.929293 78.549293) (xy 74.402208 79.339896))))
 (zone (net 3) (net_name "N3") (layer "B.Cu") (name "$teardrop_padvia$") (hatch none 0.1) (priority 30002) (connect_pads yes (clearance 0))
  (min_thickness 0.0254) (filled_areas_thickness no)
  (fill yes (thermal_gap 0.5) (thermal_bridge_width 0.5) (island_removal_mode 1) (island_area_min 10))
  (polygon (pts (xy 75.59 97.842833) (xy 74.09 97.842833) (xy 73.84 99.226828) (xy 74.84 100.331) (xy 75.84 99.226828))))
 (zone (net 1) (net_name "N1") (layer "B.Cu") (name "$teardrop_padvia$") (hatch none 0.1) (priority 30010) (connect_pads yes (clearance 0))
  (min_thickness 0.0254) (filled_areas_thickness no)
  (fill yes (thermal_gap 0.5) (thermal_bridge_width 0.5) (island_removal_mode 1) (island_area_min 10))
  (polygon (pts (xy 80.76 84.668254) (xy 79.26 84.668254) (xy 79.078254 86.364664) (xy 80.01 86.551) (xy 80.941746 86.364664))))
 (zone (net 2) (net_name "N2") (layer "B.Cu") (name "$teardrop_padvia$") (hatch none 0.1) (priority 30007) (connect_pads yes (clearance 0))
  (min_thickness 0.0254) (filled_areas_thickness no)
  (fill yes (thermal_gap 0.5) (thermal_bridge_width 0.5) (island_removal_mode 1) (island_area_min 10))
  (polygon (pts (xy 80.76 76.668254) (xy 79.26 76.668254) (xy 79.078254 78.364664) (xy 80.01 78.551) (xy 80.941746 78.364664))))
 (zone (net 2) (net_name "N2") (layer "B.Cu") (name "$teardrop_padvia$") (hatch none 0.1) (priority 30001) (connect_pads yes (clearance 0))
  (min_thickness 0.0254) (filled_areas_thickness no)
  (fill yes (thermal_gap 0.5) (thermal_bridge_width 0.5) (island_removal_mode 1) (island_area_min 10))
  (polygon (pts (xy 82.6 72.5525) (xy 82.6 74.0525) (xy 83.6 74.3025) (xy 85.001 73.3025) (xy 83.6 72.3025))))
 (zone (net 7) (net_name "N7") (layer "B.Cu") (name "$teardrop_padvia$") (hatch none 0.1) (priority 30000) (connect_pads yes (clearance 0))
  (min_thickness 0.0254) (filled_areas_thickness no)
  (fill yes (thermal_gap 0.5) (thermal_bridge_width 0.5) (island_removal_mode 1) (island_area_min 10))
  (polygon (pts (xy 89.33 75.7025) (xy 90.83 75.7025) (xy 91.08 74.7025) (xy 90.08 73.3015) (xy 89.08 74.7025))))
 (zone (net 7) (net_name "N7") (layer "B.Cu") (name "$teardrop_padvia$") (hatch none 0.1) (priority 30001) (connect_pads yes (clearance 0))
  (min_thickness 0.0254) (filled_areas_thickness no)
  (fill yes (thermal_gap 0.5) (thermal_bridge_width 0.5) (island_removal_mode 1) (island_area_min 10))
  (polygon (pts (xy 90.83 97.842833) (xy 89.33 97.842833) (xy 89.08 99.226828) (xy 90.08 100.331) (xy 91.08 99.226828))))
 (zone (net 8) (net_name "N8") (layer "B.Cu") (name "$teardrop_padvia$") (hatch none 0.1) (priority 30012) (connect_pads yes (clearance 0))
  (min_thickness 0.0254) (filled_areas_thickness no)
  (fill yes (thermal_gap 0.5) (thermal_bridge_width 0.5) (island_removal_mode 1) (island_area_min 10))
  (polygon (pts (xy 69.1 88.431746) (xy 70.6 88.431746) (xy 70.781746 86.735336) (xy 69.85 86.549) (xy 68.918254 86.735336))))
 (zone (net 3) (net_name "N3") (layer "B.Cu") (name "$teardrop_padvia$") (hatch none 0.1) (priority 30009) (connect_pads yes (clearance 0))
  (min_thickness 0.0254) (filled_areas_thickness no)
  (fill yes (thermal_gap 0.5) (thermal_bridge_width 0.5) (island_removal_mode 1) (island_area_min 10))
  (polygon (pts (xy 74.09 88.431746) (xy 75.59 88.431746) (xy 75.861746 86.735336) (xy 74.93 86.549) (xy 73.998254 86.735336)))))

